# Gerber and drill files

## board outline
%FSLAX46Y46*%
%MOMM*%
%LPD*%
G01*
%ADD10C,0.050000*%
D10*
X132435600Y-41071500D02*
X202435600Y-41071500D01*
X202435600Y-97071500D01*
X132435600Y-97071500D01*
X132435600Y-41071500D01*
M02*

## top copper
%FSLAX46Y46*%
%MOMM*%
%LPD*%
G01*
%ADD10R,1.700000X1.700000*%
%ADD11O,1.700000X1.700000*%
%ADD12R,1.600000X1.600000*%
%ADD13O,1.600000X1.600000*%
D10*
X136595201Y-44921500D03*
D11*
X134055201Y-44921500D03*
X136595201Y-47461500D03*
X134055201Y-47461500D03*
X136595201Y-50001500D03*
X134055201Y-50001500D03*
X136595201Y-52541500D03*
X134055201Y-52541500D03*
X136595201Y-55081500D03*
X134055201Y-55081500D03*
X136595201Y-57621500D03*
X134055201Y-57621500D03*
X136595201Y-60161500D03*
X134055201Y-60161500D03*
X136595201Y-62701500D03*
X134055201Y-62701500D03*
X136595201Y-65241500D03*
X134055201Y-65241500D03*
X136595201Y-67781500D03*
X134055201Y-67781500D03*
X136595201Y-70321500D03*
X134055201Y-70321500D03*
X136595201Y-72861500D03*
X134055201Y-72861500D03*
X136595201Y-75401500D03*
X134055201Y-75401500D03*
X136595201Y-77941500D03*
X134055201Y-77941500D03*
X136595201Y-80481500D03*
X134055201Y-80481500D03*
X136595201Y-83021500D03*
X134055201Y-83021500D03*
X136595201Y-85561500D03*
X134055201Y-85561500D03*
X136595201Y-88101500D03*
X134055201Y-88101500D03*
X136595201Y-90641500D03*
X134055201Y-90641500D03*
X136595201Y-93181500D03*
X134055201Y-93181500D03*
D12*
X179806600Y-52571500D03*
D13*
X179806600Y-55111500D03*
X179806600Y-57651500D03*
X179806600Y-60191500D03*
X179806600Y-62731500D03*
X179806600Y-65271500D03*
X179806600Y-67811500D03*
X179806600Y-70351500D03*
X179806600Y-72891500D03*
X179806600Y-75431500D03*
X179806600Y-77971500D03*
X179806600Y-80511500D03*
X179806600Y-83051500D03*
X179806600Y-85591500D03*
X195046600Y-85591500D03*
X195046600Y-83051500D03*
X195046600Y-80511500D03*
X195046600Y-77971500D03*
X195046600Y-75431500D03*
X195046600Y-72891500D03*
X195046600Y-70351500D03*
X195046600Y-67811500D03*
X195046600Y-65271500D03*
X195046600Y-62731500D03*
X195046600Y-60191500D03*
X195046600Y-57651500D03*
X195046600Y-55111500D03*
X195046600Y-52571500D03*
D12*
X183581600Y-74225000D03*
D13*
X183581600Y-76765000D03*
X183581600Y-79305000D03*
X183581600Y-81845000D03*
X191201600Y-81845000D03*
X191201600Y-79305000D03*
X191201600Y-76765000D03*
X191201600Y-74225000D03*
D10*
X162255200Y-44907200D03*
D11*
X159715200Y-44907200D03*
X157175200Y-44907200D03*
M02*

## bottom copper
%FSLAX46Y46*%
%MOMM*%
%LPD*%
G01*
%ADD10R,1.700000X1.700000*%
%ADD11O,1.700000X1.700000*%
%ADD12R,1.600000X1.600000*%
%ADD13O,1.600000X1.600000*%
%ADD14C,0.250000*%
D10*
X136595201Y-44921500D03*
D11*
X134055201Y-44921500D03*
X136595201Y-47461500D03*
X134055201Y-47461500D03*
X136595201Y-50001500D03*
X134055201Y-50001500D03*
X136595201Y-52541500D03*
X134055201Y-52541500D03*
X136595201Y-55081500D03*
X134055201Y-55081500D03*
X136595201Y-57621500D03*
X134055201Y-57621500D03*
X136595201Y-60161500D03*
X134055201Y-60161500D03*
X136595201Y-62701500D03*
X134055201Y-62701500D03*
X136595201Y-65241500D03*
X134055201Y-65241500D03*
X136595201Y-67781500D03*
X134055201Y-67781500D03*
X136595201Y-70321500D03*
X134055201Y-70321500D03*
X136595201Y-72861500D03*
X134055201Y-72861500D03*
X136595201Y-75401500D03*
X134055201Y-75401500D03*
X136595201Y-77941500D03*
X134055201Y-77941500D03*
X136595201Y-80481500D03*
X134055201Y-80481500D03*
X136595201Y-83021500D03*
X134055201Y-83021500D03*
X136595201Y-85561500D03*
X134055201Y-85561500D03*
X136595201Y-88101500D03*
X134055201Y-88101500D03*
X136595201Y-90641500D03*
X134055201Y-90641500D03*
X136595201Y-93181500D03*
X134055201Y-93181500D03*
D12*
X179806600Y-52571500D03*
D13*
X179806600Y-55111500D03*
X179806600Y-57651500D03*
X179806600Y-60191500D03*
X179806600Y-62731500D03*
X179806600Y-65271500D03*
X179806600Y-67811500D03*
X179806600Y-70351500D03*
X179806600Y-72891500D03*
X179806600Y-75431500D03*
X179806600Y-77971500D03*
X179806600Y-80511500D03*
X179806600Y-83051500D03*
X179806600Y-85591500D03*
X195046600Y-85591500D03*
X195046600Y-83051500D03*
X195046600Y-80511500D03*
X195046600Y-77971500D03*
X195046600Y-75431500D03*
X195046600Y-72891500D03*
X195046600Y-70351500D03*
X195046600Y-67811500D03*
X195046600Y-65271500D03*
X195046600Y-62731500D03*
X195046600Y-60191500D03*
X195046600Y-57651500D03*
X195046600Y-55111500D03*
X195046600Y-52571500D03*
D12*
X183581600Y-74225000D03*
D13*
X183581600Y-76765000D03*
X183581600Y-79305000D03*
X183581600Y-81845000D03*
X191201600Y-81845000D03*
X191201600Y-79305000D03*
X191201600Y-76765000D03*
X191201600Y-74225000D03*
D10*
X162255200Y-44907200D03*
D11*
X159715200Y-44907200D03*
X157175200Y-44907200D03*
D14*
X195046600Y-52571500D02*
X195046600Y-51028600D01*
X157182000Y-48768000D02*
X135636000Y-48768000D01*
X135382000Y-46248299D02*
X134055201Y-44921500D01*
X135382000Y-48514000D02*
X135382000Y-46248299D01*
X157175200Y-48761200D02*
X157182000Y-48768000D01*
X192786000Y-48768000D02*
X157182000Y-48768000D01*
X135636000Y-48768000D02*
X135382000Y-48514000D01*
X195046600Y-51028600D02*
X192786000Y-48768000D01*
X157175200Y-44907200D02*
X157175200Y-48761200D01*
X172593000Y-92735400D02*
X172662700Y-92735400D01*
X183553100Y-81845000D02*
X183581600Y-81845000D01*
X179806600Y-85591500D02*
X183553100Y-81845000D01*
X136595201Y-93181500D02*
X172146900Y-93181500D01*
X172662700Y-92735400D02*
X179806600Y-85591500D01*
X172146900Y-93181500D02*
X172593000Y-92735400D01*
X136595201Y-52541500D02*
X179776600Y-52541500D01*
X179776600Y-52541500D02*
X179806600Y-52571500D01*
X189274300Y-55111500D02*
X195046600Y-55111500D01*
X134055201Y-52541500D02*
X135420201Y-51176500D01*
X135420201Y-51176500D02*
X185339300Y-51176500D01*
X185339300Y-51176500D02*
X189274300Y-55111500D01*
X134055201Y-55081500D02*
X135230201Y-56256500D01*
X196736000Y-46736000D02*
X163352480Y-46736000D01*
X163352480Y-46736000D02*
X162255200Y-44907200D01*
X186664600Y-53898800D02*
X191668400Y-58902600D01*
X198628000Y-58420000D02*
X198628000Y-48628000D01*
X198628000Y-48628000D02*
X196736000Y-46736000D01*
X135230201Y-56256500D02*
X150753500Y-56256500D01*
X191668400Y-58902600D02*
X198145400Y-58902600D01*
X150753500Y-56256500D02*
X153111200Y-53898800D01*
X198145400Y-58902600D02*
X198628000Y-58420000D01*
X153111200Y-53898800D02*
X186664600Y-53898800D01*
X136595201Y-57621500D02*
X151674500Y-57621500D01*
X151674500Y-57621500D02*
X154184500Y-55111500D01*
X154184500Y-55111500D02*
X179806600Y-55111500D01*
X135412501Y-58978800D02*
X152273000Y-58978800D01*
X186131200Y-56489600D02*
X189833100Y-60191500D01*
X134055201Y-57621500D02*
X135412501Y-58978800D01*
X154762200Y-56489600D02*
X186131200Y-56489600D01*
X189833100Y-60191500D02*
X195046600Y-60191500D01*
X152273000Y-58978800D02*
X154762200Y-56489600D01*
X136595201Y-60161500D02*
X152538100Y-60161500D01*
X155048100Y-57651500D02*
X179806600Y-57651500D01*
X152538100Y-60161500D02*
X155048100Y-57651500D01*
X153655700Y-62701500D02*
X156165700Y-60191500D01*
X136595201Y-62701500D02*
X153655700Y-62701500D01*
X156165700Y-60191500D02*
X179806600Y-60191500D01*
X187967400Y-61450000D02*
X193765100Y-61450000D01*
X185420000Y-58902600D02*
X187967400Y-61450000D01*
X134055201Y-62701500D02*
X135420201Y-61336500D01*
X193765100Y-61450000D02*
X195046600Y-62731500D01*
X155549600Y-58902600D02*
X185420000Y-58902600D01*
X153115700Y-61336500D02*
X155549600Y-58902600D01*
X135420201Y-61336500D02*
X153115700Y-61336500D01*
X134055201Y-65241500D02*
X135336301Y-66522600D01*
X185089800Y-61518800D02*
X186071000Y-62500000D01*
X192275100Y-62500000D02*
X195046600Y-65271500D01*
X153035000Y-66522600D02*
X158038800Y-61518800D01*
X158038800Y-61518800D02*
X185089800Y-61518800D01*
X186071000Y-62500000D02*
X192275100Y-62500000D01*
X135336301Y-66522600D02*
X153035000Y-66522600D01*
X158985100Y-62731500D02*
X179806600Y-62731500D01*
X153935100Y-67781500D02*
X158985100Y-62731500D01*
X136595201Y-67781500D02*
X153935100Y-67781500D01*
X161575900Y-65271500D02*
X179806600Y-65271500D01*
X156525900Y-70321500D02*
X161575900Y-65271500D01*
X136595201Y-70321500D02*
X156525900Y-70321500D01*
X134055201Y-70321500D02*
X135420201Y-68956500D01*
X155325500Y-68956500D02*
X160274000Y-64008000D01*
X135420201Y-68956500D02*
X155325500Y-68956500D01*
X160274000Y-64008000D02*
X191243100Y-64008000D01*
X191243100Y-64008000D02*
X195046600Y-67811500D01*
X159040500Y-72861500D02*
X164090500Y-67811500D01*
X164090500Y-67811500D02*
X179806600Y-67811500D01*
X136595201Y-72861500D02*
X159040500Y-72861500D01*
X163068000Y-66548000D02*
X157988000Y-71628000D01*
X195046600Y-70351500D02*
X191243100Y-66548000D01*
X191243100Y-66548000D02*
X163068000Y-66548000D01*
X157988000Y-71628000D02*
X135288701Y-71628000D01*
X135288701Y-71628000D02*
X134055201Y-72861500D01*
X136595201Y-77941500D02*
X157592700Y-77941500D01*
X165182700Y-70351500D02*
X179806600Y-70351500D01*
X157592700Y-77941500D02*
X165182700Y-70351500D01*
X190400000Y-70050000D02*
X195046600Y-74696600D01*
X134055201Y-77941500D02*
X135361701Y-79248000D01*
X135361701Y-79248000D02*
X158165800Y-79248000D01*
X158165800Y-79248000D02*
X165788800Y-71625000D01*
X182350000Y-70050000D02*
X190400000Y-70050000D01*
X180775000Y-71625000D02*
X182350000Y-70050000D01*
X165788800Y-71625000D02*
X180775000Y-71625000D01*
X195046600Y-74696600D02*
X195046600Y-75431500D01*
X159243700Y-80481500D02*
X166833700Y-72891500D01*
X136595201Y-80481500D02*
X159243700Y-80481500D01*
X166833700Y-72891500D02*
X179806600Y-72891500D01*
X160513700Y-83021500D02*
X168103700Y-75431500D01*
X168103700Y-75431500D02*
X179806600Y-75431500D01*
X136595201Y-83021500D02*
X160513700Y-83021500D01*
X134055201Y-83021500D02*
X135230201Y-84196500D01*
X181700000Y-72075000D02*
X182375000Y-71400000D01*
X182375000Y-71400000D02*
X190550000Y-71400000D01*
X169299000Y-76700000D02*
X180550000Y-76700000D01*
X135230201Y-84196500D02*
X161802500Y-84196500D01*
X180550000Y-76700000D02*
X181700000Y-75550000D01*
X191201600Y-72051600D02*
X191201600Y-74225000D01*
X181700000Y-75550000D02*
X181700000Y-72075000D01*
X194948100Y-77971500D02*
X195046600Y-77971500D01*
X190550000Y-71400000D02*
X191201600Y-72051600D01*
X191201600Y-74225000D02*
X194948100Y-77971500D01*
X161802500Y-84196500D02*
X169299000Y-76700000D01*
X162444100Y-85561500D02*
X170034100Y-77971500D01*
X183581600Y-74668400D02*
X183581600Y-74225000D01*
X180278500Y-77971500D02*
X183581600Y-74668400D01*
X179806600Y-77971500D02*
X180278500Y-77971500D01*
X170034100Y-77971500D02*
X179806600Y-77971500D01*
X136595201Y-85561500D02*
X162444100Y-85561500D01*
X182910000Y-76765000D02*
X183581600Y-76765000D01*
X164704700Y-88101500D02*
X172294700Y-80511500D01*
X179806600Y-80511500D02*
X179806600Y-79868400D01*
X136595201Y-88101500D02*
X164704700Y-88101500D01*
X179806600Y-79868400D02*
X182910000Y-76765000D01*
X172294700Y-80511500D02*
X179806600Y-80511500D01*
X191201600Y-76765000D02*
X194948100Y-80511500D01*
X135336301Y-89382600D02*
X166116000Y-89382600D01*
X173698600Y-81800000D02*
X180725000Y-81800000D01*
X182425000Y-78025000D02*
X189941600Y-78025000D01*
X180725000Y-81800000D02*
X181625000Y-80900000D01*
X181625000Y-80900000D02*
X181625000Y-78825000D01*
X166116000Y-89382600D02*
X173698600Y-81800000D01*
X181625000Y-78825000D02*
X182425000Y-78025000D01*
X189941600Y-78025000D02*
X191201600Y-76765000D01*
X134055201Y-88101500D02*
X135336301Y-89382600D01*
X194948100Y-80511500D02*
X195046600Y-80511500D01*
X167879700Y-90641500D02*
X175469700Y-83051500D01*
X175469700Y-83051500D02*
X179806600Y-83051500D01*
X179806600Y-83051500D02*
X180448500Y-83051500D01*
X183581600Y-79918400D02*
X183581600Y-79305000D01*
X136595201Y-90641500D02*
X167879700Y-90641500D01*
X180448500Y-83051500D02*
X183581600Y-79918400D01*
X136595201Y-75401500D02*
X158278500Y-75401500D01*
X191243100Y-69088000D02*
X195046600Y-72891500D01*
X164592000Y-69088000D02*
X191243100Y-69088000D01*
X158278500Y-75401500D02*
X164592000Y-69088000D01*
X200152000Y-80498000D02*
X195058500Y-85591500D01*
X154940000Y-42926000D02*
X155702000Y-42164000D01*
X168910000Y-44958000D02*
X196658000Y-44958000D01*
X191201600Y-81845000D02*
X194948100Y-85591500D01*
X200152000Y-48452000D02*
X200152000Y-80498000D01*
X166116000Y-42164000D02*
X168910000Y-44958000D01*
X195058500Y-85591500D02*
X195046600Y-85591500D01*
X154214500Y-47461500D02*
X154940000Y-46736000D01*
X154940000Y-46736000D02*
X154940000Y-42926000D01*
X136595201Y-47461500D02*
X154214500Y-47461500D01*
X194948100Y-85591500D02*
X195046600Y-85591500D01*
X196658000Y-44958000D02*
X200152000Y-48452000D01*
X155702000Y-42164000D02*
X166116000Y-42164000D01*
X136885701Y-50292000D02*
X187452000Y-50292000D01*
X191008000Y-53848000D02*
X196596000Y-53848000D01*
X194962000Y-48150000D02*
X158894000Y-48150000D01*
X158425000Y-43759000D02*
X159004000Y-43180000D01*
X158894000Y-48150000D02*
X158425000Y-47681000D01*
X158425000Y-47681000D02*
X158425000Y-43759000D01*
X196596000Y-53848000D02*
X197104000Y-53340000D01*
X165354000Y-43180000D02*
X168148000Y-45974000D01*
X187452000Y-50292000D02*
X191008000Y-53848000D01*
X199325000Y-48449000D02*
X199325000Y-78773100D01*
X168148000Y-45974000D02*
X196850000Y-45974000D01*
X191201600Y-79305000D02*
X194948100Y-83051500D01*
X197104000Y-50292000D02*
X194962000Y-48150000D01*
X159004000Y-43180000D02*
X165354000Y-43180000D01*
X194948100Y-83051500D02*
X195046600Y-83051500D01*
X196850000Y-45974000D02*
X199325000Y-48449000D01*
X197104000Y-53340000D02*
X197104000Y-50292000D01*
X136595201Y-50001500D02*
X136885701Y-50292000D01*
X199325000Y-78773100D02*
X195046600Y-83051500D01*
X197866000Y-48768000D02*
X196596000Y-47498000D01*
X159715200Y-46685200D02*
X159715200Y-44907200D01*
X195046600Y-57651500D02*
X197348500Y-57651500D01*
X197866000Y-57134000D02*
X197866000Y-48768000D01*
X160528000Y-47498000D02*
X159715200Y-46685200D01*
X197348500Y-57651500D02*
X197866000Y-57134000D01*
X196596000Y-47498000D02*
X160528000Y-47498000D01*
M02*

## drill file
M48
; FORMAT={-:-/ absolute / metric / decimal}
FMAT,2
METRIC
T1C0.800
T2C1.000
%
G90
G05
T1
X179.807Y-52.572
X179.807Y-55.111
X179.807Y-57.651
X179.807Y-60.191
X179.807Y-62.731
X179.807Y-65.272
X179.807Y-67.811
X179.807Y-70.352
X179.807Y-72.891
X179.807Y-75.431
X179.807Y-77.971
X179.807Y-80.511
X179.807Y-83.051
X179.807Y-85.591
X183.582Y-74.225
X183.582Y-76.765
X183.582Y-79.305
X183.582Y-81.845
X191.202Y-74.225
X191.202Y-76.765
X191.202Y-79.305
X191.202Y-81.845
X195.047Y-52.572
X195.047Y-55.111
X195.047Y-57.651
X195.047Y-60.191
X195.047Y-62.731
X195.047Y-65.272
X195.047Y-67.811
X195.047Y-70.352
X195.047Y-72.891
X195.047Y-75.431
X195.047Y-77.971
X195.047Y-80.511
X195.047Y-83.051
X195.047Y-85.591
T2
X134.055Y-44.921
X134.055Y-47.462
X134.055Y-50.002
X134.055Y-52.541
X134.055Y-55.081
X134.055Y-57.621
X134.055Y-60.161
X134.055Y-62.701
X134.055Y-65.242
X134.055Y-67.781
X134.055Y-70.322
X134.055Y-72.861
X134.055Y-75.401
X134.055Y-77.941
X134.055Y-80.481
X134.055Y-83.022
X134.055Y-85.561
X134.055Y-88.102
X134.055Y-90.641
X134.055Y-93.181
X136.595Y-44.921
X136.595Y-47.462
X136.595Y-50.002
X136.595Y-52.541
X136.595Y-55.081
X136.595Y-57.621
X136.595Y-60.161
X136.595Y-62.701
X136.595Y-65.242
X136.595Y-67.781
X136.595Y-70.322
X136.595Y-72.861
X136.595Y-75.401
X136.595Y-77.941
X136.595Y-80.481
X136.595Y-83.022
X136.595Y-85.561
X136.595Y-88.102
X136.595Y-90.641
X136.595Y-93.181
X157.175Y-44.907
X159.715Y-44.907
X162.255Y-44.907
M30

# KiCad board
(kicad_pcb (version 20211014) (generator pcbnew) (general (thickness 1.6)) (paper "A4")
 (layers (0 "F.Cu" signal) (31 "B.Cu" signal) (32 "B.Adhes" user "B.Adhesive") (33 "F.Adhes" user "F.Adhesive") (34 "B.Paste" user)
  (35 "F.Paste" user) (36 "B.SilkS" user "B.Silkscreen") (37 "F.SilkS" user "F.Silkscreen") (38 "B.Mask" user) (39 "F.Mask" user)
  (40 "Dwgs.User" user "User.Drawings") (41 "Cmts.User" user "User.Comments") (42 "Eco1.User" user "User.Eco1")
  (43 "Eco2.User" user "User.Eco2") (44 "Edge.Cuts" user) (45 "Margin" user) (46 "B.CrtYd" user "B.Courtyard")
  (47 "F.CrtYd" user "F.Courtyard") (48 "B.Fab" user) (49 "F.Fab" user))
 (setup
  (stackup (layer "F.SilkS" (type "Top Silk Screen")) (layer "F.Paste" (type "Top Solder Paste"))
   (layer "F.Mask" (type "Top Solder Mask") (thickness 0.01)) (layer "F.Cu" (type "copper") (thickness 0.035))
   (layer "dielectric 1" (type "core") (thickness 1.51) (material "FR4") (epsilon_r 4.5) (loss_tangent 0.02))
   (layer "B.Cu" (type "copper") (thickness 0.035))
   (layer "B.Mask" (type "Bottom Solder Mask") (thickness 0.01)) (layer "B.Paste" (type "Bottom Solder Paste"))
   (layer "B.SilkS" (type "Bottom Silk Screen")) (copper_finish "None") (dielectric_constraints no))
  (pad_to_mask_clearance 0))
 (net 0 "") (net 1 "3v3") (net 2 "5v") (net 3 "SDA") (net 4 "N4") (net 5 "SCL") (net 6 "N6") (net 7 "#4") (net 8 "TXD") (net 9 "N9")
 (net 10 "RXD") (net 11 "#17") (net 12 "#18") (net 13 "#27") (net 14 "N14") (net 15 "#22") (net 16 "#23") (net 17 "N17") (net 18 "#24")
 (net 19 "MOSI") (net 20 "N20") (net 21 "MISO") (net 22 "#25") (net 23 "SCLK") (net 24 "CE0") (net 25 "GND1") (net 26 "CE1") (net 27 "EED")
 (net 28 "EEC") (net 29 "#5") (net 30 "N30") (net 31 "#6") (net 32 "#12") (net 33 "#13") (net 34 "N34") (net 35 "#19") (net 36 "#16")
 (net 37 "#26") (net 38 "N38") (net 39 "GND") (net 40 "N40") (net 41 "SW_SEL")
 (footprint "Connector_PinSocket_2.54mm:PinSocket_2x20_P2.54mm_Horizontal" (layer "F.Cu") (at 136.595201 44.9215)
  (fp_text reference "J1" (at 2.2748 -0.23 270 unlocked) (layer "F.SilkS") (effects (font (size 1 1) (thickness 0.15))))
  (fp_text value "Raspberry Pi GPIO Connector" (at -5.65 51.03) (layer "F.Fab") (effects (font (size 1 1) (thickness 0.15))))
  (pad "1" thru_hole rect (at 0 0) (size 1.7 1.7) (drill 1) (layers *.Cu *.Mask) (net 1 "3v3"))
  (pad "2" thru_hole oval (at -2.54 0) (size 1.7 1.7) (drill 1) (layers *.Cu *.Mask) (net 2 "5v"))
  (pad "3" thru_hole oval (at 0 2.54) (size 1.7 1.7) (drill 1) (layers *.Cu *.Mask) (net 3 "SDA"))
  (pad "4" thru_hole oval (at -2.54 2.54) (size 1.7 1.7) (drill 1) (layers *.Cu *.Mask) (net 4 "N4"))
  (pad "5" thru_hole oval (at 0 5.08) (size 1.7 1.7) (drill 1) (layers *.Cu *.Mask) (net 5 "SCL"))
  (pad "6" thru_hole oval (at -2.54 5.08) (size 1.7 1.7) (drill 1) (layers *.Cu *.Mask) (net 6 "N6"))
  (pad "7" thru_hole oval (at 0 7.62) (size 1.7 1.7) (drill 1) (layers *.Cu *.Mask) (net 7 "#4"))
  (pad "8" thru_hole oval (at -2.54 7.62) (size 1.7 1.7) (drill 1) (layers *.Cu *.Mask) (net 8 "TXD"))
  (pad "9" thru_hole oval (at 0 10.16) (size 1.7 1.7) (drill 1) (layers *.Cu *.Mask) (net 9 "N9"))
  (pad "10" thru_hole oval (at -2.54 10.16) (size 1.7 1.7) (drill 1) (layers *.Cu *.Mask) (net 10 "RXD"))
  (pad "11" thru_hole oval (at 0 12.7) (size 1.7 1.7) (drill 1) (layers *.Cu *.Mask) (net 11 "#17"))
  (pad "12" thru_hole oval (at -2.54 12.7) (size 1.7 1.7) (drill 1) (layers *.Cu *.Mask) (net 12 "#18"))
  (pad "13" thru_hole oval (at 0 15.24) (size 1.7 1.7) (drill 1) (layers *.Cu *.Mask) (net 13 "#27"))
  (pad "14" thru_hole oval (at -2.54 15.24) (size 1.7 1.7) (drill 1) (layers *.Cu *.Mask) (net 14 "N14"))
  (pad "15" thru_hole oval (at 0 17.78) (size 1.7 1.7) (drill 1) (layers *.Cu *.Mask) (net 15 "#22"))
  (pad "16" thru_hole oval (at -2.54 17.78) (size 1.7 1.7) (drill 1) (layers *.Cu *.Mask) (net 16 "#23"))
  (pad "17" thru_hole oval (at 0 20.32) (size 1.7 1.7) (drill 1) (layers *.Cu *.Mask) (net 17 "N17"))
  (pad "18" thru_hole oval (at -2.54 20.32) (size 1.7 1.7) (drill 1) (layers *.Cu *.Mask) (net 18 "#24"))
  (pad "19" thru_hole oval (at 0 22.86) (size 1.7 1.7) (drill 1) (layers *.Cu *.Mask) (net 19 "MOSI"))
  (pad "20" thru_hole oval (at -2.54 22.86) (size 1.7 1.7) (drill 1) (layers *.Cu *.Mask) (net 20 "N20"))
  (pad "21" thru_hole oval (at 0 25.4) (size 1.7 1.7) (drill 1) (layers *.Cu *.Mask) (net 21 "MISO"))
  (pad "22" thru_hole oval (at -2.54 25.4) (size 1.7 1.7) (drill 1) (layers *.Cu *.Mask) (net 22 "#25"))
  (pad "23" thru_hole oval (at 0 27.94) (size 1.7 1.7) (drill 1) (layers *.Cu *.Mask) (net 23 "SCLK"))
  (pad "24" thru_hole oval (at -2.54 27.94) (size 1.7 1.7) (drill 1) (layers *.Cu *.Mask) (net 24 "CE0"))
  (pad "25" thru_hole oval (at 0 30.48) (size 1.7 1.7) (drill 1) (layers *.Cu *.Mask) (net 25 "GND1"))
  (pad "26" thru_hole oval (at -2.54 30.48) (size 1.7 1.7) (drill 1) (layers *.Cu *.Mask) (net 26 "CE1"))
  (pad "27" thru_hole oval (at 0 33.02) (size 1.7 1.7) (drill 1) (layers *.Cu *.Mask) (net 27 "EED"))
  (pad "28" thru_hole oval (at -2.54 33.02) (size 1.7 1.7) (drill 1) (layers *.Cu *.Mask) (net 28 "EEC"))
  (pad "29" thru_hole oval (at 0 35.56) (size 1.7 1.7) (drill 1) (layers *.Cu *.Mask) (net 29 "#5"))
  (pad "30" thru_hole oval (at -2.54 35.56) (size 1.7 1.7) (drill 1) (layers *.Cu *.Mask) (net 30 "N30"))
  (pad "31" thru_hole oval (at 0 38.1) (size 1.7 1.7) (drill 1) (layers *.Cu *.Mask) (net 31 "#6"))
  (pad "32" thru_hole oval (at -2.54 38.1) (size 1.7 1.7) (drill 1) (layers *.Cu *.Mask) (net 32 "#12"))
  (pad "33" thru_hole oval (at 0 40.64) (size 1.7 1.7) (drill 1) (layers *.Cu *.Mask) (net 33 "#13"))
  (pad "34" thru_hole oval (at -2.54 40.64) (size 1.7 1.7) (drill 1) (layers *.Cu *.Mask) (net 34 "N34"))
  (pad "35" thru_hole oval (at 0 43.18) (size 1.7 1.7) (drill 1) (layers *.Cu *.Mask) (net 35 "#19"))
  (pad "36" thru_hole oval (at -2.54 43.18) (size 1.7 1.7) (drill 1) (layers *.Cu *.Mask) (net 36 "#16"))
  (pad "37" thru_hole oval (at 0 45.72) (size 1.7 1.7) (drill 1) (layers *.Cu *.Mask) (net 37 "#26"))
  (pad "38" thru_hole oval (at -2.54 45.72) (size 1.7 1.7) (drill 1) (layers *.Cu *.Mask) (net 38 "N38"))
  (pad "39" thru_hole oval (at 0 48.26) (size 1.7 1.7) (drill 1) (layers *.Cu *.Mask) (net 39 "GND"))
  (pad "40" thru_hole oval (at -2.54 48.26) (size 1.7 1.7) (drill 1) (layers *.Cu *.Mask) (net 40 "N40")))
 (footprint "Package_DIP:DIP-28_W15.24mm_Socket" (layer "F.Cu") (at 179.8066 52.5715)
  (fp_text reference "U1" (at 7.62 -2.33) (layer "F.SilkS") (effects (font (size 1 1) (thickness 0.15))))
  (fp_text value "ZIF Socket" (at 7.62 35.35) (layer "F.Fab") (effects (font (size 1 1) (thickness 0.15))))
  (pad "1" thru_hole rect (at 0 0) (size 1.6 1.6) (drill 0.8) (layers *.Cu *.Mask) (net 7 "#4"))
  (pad "2" thru_hole oval (at 0 2.54) (size 1.6 1.6) (drill 0.8) (layers *.Cu *.Mask) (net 11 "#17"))
  (pad "3" thru_hole oval (at 0 5.08) (size 1.6 1.6) (drill 0.8) (layers *.Cu *.Mask) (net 13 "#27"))
  (pad "4" thru_hole oval (at 0 7.62) (size 1.6 1.6) (drill 0.8) (layers *.Cu *.Mask) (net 15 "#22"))
  (pad "5" thru_hole oval (at 0 10.16) (size 1.6 1.6) (drill 0.8) (layers *.Cu *.Mask) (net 19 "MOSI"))
  (pad "6" thru_hole oval (at 0 12.7) (size 1.6 1.6) (drill 0.8) (layers *.Cu *.Mask) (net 21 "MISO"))
  (pad "7" thru_hole oval (at 0 15.24) (size 1.6 1.6) (drill 0.8) (layers *.Cu *.Mask) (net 23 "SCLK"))
  (pad "8" thru_hole oval (at 0 17.78) (size 1.6 1.6) (drill 0.8) (layers *.Cu *.Mask) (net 27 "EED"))
  (pad "9" thru_hole oval (at 0 20.32) (size 1.6 1.6) (drill 0.8) (layers *.Cu *.Mask) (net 29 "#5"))
  (pad "10" thru_hole oval (at 0 22.86) (size 1.6 1.6) (drill 0.8) (layers *.Cu *.Mask) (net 31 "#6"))
  (pad "11" thru_hole oval (at 0 25.4) (size 1.6 1.6) (drill 0.8) (layers *.Cu *.Mask) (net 33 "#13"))
  (pad "12" thru_hole oval (at 0 27.94) (size 1.6 1.6) (drill 0.8) (layers *.Cu *.Mask) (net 35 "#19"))
  (pad "13" thru_hole oval (at 0 30.48) (size 1.6 1.6) (drill 0.8) (layers *.Cu *.Mask) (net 37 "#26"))
  (pad "14" thru_hole oval (at 0 33.02) (size 1.6 1.6) (drill 0.8) (layers *.Cu *.Mask) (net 39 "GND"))
  (pad "15" thru_hole oval (at 15.24 33.02) (size 1.6 1.6) (drill 0.8) (layers *.Cu *.Mask) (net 3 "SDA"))
  (pad "16" thru_hole oval (at 15.24 30.48) (size 1.6 1.6) (drill 0.8) (layers *.Cu *.Mask) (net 5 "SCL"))
  (pad "17" thru_hole oval (at 15.24 27.94) (size 1.6 1.6) (drill 0.8) (layers *.Cu *.Mask) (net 36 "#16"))
  (pad "18" thru_hole oval (at 15.24 25.4) (size 1.6 1.6) (drill 0.8) (layers *.Cu *.Mask) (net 32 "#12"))
  (pad "19" thru_hole oval (at 15.24 22.86) (size 1.6 1.6) (drill 0.8) (layers *.Cu *.Mask) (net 28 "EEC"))
  (pad "20" thru_hole oval (at 15.24 20.32) (size 1.6 1.6) (drill 0.8) (layers *.Cu *.Mask) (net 25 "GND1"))
  (pad "21" thru_hole oval (at 15.24 17.78) (size 1.6 1.6) (drill 0.8) (layers *.Cu *.Mask) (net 24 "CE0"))
  (pad "22" thru_hole oval (at 15.24 15.24) (size 1.6 1.6) (drill 0.8) (layers *.Cu *.Mask) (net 22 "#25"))
  (pad "23" thru_hole oval (at 15.24 12.7) (size 1.6 1.6) (drill 0.8) (layers *.Cu *.Mask) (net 18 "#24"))
  (pad "24" thru_hole oval (at 15.24 10.16) (size 1.6 1.6) (drill 0.8) (layers *.Cu *.Mask) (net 16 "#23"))
  (pad "25" thru_hole oval (at 15.24 7.62) (size 1.6 1.6) (drill 0.8) (layers *.Cu *.Mask) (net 12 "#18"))
  (pad "26" thru_hole oval (at 15.24 5.08) (size 1.6 1.6) (drill 0.8) (layers *.Cu *.Mask) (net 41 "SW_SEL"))
  (pad "27" thru_hole oval (at 15.24 2.54) (size 1.6 1.6) (drill 0.8) (layers *.Cu *.Mask) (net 8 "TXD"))
  (pad "28" thru_hole oval (at 15.24 0) (size 1.6 1.6) (drill 0.8) (layers *.Cu *.Mask) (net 2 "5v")))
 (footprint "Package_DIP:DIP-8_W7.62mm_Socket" (layer "F.Cu") (at 183.5816 74.225)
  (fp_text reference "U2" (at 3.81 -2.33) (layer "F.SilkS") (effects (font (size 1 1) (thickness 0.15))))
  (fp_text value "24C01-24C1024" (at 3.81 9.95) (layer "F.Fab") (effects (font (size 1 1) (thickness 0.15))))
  (pad "1" thru_hole rect (at 0 0) (size 1.6 1.6) (drill 0.8) (layers *.Cu *.Mask) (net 33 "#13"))
  (pad "2" thru_hole oval (at 0 2.54) (size 1.6 1.6) (drill 0.8) (layers *.Cu *.Mask) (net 35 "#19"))
  (pad "3" thru_hole oval (at 0 5.08) (size 1.6 1.6) (drill 0.8) (layers *.Cu *.Mask) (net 37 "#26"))
  (pad "4" thru_hole oval (at 0 7.62) (size 1.6 1.6) (drill 0.8) (layers *.Cu *.Mask) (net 39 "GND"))
  (pad "5" thru_hole oval (at 7.62 7.62) (size 1.6 1.6) (drill 0.8) (layers *.Cu *.Mask) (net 3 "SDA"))
  (pad "6" thru_hole oval (at 7.62 5.08) (size 1.6 1.6) (drill 0.8) (layers *.Cu *.Mask) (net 5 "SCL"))
  (pad "7" thru_hole oval (at 7.62 2.54) (size 1.6 1.6) (drill 0.8) (layers *.Cu *.Mask) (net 36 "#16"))
  (pad "8" thru_hole oval (at 7.62 0) (size 1.6 1.6) (drill 0.8) (layers *.Cu *.Mask) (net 32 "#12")))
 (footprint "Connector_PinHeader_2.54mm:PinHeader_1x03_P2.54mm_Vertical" (layer "F.Cu") (at 162.2552 44.9072 -90)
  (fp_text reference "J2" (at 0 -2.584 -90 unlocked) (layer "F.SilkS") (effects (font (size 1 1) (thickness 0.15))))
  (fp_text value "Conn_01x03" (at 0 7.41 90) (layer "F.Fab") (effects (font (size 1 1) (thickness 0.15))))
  (pad "1" thru_hole rect (at 0 0 270) (size 1.7 1.7) (drill 1) (layers *.Cu *.Mask) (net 10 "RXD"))
  (pad "2" thru_hole oval (at 0 2.54 270) (size 1.7 1.7) (drill 1) (layers *.Cu *.Mask) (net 41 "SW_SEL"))
  (pad "3" thru_hole oval (at 0 5.08 270) (size 1.7 1.7) (drill 1) (layers *.Cu *.Mask) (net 2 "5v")))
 (gr_rect (start 132.4356 41.0715) (end 202.4356 97.0715) (layer "Edge.Cuts") (width 0.05) (fill none))
 (segment (start 195.0466 52.5715) (end 195.0466 51.0286) (width 0.25) (layer "B.Cu") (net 2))
 (segment (start 157.182 48.768) (end 135.636 48.768) (width 0.25) (layer "B.Cu") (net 2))
 (segment (start 135.382 46.248299) (end 134.055201 44.9215) (width 0.25) (layer "B.Cu") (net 2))
 (segment (start 135.382 48.514) (end 135.382 46.248299) (width 0.25) (layer "B.Cu") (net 2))
 (segment (start 157.1752 48.7612) (end 157.182 48.768) (width 0.25) (layer "B.Cu") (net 2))
 (segment (start 192.786 48.768) (end 157.182 48.768) (width 0.25) (layer "B.Cu") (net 2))
 (segment (start 135.636 48.768) (end 135.382 48.514) (width 0.25) (layer "B.Cu") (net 2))
 (segment (start 195.0466 51.0286) (end 192.786 48.768) (width 0.25) (layer "B.Cu") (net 2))
 (segment (start 157.1752 44.9072) (end 157.1752 48.7612) (width 0.25) (layer "B.Cu") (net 2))
 (segment (start 172.593 92.7354) (end 172.6627 92.7354) (width 0.25) (layer "B.Cu") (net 39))
 (segment (start 183.5531 81.845) (end 183.5816 81.845) (width 0.25) (layer "B.Cu") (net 39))
 (segment (start 179.8066 85.5915) (end 183.5531 81.845) (width 0.25) (layer "B.Cu") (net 39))
 (segment (start 136.595201 93.1815) (end 172.1469 93.1815) (width 0.25) (layer "B.Cu") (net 39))
 (segment (start 172.6627 92.7354) (end 179.8066 85.5915) (width 0.25) (layer "B.Cu") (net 39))
 (segment (start 172.1469 93.1815) (end 172.593 92.7354) (width 0.25) (layer "B.Cu") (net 39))
 (segment (start 136.595201 52.5415) (end 179.7766 52.5415) (width 0.25) (layer "B.Cu") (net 7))
 (segment (start 179.7766 52.5415) (end 179.8066 52.5715) (width 0.25) (layer "B.Cu") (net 7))
 (segment (start 189.2743 55.1115) (end 195.0466 55.1115) (width 0.25) (layer "B.Cu") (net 8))
 (segment (start 134.055201 52.5415) (end 135.420201 51.1765) (width 0.25) (layer "B.Cu") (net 8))
 (segment (start 135.420201 51.1765) (end 185.3393 51.1765) (width 0.25) (layer "B.Cu") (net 8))
 (segment (start 185.3393 51.1765) (end 189.2743 55.1115) (width 0.25) (layer "B.Cu") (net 8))
 (segment (start 134.055201 55.0815) (end 135.230201 56.2565) (width 0.25) (layer "B.Cu") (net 10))
 (segment (start 196.736 46.736) (end 163.35248 46.736) (width 0.25) (layer "B.Cu") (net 10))
 (segment (start 163.35248 46.736) (end 162.2552 44.9072) (width 0.25) (layer "B.Cu") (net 10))
 (segment (start 186.6646 53.8988) (end 191.6684 58.9026) (width 0.25) (layer "B.Cu") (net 10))
 (segment (start 198.628 58.42) (end 198.628 48.628) (width 0.25) (layer "B.Cu") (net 10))
 (segment (start 198.628 48.628) (end 196.736 46.736) (width 0.25) (layer "B.Cu") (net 10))
 (segment (start 135.230201 56.2565) (end 150.7535 56.2565) (width 0.25) (layer "B.Cu") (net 10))
 (segment (start 191.6684 58.9026) (end 198.1454 58.9026) (width 0.25) (layer "B.Cu") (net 10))
 (segment (start 150.7535 56.2565) (end 153.1112 53.8988) (width 0.25) (layer "B.Cu") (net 10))
 (segment (start 198.1454 58.9026) (end 198.628 58.42) (width 0.25) (layer "B.Cu") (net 10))
 (segment (start 153.1112 53.8988) (end 186.6646 53.8988) (width 0.25) (layer "B.Cu") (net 10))
 (segment (start 136.595201 57.6215) (end 151.6745 57.6215) (width 0.25) (layer "B.Cu") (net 11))
 (segment (start 151.6745 57.6215) (end 154.1845 55.1115) (width 0.25) (layer "B.Cu") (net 11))
 (segment (start 154.1845 55.1115) (end 179.8066 55.1115) (width 0.25) (layer "B.Cu") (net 11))
 (segment (start 135.412501 58.9788) (end 152.273 58.9788) (width 0.25) (layer "B.Cu") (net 12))
 (segment (start 186.1312 56.4896) (end 189.8331 60.1915) (width 0.25) (layer "B.Cu") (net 12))
 (segment (start 134.055201 57.6215) (end 135.412501 58.9788) (width 0.25) (layer "B.Cu") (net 12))
 (segment (start 154.7622 56.4896) (end 186.1312 56.4896) (width 0.25) (layer "B.Cu") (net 12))
 (segment (start 189.8331 60.1915) (end 195.0466 60.1915) (width 0.25) (layer "B.Cu") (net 12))
 (segment (start 152.273 58.9788) (end 154.7622 56.4896) (width 0.25) (layer "B.Cu") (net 12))
 (segment (start 136.595201 60.1615) (end 152.5381 60.1615) (width 0.25) (layer "B.Cu") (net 13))
 (segment (start 155.0481 57.6515) (end 179.8066 57.6515) (width 0.25) (layer "B.Cu") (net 13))
 (segment (start 152.5381 60.1615) (end 155.0481 57.6515) (width 0.25) (layer "B.Cu") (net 13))
 (segment (start 153.6557 62.7015) (end 156.1657 60.1915) (width 0.25) (layer "B.Cu") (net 15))
 (segment (start 136.595201 62.7015) (end 153.6557 62.7015) (width 0.25) (layer "B.Cu") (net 15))
 (segment (start 156.1657 60.1915) (end 179.8066 60.1915) (width 0.25) (layer "B.Cu") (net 15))
 (segment (start 187.9674 61.45) (end 193.7651 61.45) (width 0.25) (layer "B.Cu") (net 16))
 (segment (start 185.42 58.9026) (end 187.9674 61.45) (width 0.25) (layer "B.Cu") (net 16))
 (segment (start 134.055201 62.7015) (end 135.420201 61.3365) (width 0.25) (layer "B.Cu") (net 16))
 (segment (start 193.7651 61.45) (end 195.0466 62.7315) (width 0.25) (layer "B.Cu") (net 16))
 (segment (start 155.5496 58.9026) (end 185.42 58.9026) (width 0.25) (layer "B.Cu") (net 16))
 (segment (start 153.1157 61.3365) (end 155.5496 58.9026) (width 0.25) (layer "B.Cu") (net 16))
 (segment (start 135.420201 61.3365) (end 153.1157 61.3365) (width 0.25) (layer "B.Cu") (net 16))
 (segment (start 134.055201 65.2415) (end 135.336301 66.5226) (width 0.25) (layer "B.Cu") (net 18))
 (segment (start 185.0898 61.5188) (end 186.071 62.5) (width 0.25) (layer "B.Cu") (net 18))
 (segment (start 192.2751 62.5) (end 195.0466 65.2715) (width 0.25) (layer "B.Cu") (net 18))
 (segment (start 153.035 66.5226) (end 158.0388 61.5188) (width 0.25) (layer "B.Cu") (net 18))
 (segment (start 158.0388 61.5188) (end 185.0898 61.5188) (width 0.25) (layer "B.Cu") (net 18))
 (segment (start 186.071 62.5) (end 192.2751 62.5) (width 0.25) (layer "B.Cu") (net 18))
 (segment (start 135.336301 66.5226) (end 153.035 66.5226) (width 0.25) (layer "B.Cu") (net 18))
 (segment (start 158.9851 62.7315) (end 179.8066 62.7315) (width 0.25) (layer "B.Cu") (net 19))
 (segment (start 153.9351 67.7815) (end 158.9851 62.7315) (width 0.25) (layer "B.Cu") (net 19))
 (segment (start 136.595201 67.7815) (end 153.9351 67.7815) (width 0.25) (layer "B.Cu") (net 19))
 (segment (start 161.5759 65.2715) (end 179.8066 65.2715) (width 0.25) (layer "B.Cu") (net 21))
 (segment (start 156.5259 70.3215) (end 161.5759 65.2715) (width 0.25) (layer "B.Cu") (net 21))
 (segment (start 136.595201 70.3215) (end 156.5259 70.3215) (width 0.25) (layer "B.Cu") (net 21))
 (segment (start 134.055201 70.3215) (end 135.420201 68.9565) (width 0.25) (layer "B.Cu") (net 22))
 (segment (start 155.3255 68.9565) (end 160.274 64.008) (width 0.25) (layer "B.Cu") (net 22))
 (segment (start 135.420201 68.9565) (end 155.3255 68.9565) (width 0.25) (layer "B.Cu") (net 22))
 (segment (start 160.274 64.008) (end 191.2431 64.008) (width 0.25) (layer "B.Cu") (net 22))
 (segment (start 191.2431 64.008) (end 195.0466 67.8115) (width 0.25) (layer "B.Cu") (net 22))
 (segment (start 159.0405 72.8615) (end 164.0905 67.8115) (width 0.25) (layer "B.Cu") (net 23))
 (segment (start 164.0905 67.8115) (end 179.8066 67.8115) (width 0.25) (layer "B.Cu") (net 23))
 (segment (start 136.595201 72.8615) (end 159.0405 72.8615) (width 0.25) (layer "B.Cu") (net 23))
 (segment (start 163.068 66.548) (end 157.988 71.628) (width 0.25) (layer "B.Cu") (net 24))
 (segment (start 195.0466 70.3515) (end 191.2431 66.548) (width 0.25) (layer "B.Cu") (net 24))
 (segment (start 191.2431 66.548) (end 163.068 66.548) (width 0.25) (layer "B.Cu") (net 24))
 (segment (start 157.988 71.628) (end 135.288701 71.628) (width 0.25) (layer "B.Cu") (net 24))
 (segment (start 135.288701 71.628) (end 134.055201 72.8615) (width 0.25) (layer "B.Cu") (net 24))
 (segment (start 136.595201 77.9415) (end 157.5927 77.9415) (width 0.25) (layer "B.Cu") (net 27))
 (segment (start 165.1827 70.3515) (end 179.8066 70.3515) (width 0.25) (layer "B.Cu") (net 27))
 (segment (start 157.5927 77.9415) (end 165.1827 70.3515) (width 0.25) (layer "B.Cu") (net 27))
 (segment (start 190.4 70.05) (end 195.0466 74.6966) (width 0.25) (layer "B.Cu") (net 28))
 (segment (start 134.055201 77.9415) (end 135.361701 79.248) (width 0.25) (layer "B.Cu") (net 28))
 (segment (start 135.361701 79.248) (end 158.1658 79.248) (width 0.25) (layer "B.Cu") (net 28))
 (segment (start 158.1658 79.248) (end 165.7888 71.625) (width 0.25) (layer "B.Cu") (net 28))
 (segment (start 182.35 70.05) (end 190.4 70.05) (width 0.25) (layer "B.Cu") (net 28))
 (segment (start 180.775 71.625) (end 182.35 70.05) (width 0.25) (layer "B.Cu") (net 28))
 (segment (start 165.7888 71.625) (end 180.775 71.625) (width 0.25) (layer "B.Cu") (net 28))
 (segment (start 195.0466 74.6966) (end 195.0466 75.4315) (width 0.25) (layer "B.Cu") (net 28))
 (segment (start 159.2437 80.4815) (end 166.8337 72.8915) (width 0.25) (layer "B.Cu") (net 29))
 (segment (start 136.595201 80.4815) (end 159.2437 80.4815) (width 0.25) (layer "B.Cu") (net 29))
 (segment (start 166.8337 72.8915) (end 179.8066 72.8915) (width 0.25) (layer "B.Cu") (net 29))
 (segment (start 160.5137 83.0215) (end 168.1037 75.4315) (width 0.25) (layer "B.Cu") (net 31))
 (segment (start 168.1037 75.4315) (end 179.8066 75.4315) (width 0.25) (layer "B.Cu") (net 31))
 (segment (start 136.595201 83.0215) (end 160.5137 83.0215) (width 0.25) (layer "B.Cu") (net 31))
 (segment (start 134.055201 83.0215) (end 135.230201 84.1965) (width 0.25) (layer "B.Cu") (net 32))
 (segment (start 181.7 72.075) (end 182.375 71.4) (width 0.25) (layer "B.Cu") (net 32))
 (segment (start 182.375 71.4) (end 190.55 71.4) (width 0.25) (layer "B.Cu") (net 32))
 (segment (start 169.299 76.7) (end 180.55 76.7) (width 0.25) (layer "B.Cu") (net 32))
 (segment (start 135.230201 84.1965) (end 161.8025 84.1965) (width 0.25) (layer "B.Cu") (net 32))
 (segment (start 180.55 76.7) (end 181.7 75.55) (width 0.25) (layer "B.Cu") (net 32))
 (segment (start 191.2016 72.0516) (end 191.2016 74.225) (width 0.25) (layer "B.Cu") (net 32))
 (segment (start 181.7 75.55) (end 181.7 72.075) (width 0.25) (layer "B.Cu") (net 32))
 (segment (start 194.9481 77.9715) (end 195.0466 77.9715) (width 0.25) (layer "B.Cu") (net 32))
 (segment (start 190.55 71.4) (end 191.2016 72.0516) (width 0.25) (layer "B.Cu") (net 32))
 (segment (start 191.2016 74.225) (end 194.9481 77.9715) (width 0.25) (layer "B.Cu") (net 32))
 (segment (start 161.8025 84.1965) (end 169.299 76.7) (width 0.25) (layer "B.Cu") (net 32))
 (segment (start 162.4441 85.5615) (end 170.0341 77.9715) (width 0.25) (layer "B.Cu") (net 33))
 (segment (start 183.5816 74.6684) (end 183.5816 74.225) (width 0.25) (layer "B.Cu") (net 33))
 (segment (start 180.2785 77.9715) (end 183.5816 74.6684) (width 0.25) (layer "B.Cu") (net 33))
 (segment (start 179.8066 77.9715) (end 180.2785 77.9715) (width 0.25) (layer "B.Cu") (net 33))
 (segment (start 170.0341 77.9715) (end 179.8066 77.9715) (width 0.25) (layer "B.Cu") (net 33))
 (segment (start 136.595201 85.5615) (end 162.4441 85.5615) (width 0.25) (layer "B.Cu") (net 33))
 (segment (start 182.91 76.765) (end 183.5816 76.765) (width 0.25) (layer "B.Cu") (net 35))
 (segment (start 164.7047 88.1015) (end 172.2947 80.5115) (width 0.25) (layer "B.Cu") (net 35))
 (segment (start 179.8066 80.5115) (end 179.8066 79.8684) (width 0.25) (layer "B.Cu") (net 35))
 (segment (start 136.595201 88.1015) (end 164.7047 88.1015) (width 0.25) (layer "B.Cu") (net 35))
 (segment (start 179.8066 79.8684) (end 182.91 76.765) (width 0.25) (layer "B.Cu") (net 35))
 (segment (start 172.2947 80.5115) (end 179.8066 80.5115) (width 0.25) (layer "B.Cu") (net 35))
 (segment (start 191.2016 76.765) (end 194.9481 80.5115) (width 0.25) (layer "B.Cu") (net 36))
 (segment (start 135.336301 89.3826) (end 166.116 89.3826) (width 0.25) (layer "B.Cu") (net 36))
 (segment (start 173.6986 81.8) (end 180.725 81.8) (width 0.25) (layer "B.Cu") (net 36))
 (segment (start 182.425 78.025) (end 189.9416 78.025) (width 0.25) (layer "B.Cu") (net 36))
 (segment (start 180.725 81.8) (end 181.625 80.9) (width 0.25) (layer "B.Cu") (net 36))
 (segment (start 181.625 80.9) (end 181.625 78.825) (width 0.25) (layer "B.Cu") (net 36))
 (segment (start 166.116 89.3826) (end 173.6986 81.8) (width 0.25) (layer "B.Cu") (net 36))
 (segment (start 181.625 78.825) (end 182.425 78.025) (width 0.25) (layer "B.Cu") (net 36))
 (segment (start 189.9416 78.025) (end 191.2016 76.765) (width 0.25) (layer "B.Cu") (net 36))
 (segment (start 134.055201 88.1015) (end 135.336301 89.3826) (width 0.25) (layer "B.Cu") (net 36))
 (segment (start 194.9481 80.5115) (end 195.0466 80.5115) (width 0.25) (layer "B.Cu") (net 36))
 (segment (start 167.8797 90.6415) (end 175.4697 83.0515) (width 0.25) (layer "B.Cu") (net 37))
 (segment (start 175.4697 83.0515) (end 179.8066 83.0515) (width 0.25) (layer "B.Cu") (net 37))
 (segment (start 179.8066 83.0515) (end 180.4485 83.0515) (width 0.25) (layer "B.Cu") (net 37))
 (segment (start 183.5816 79.9184) (end 183.5816 79.305) (width 0.25) (layer "B.Cu") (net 37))
 (segment (start 136.595201 90.6415) (end 167.8797 90.6415) (width 0.25) (layer "B.Cu") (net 37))
 (segment (start 180.4485 83.0515) (end 183.5816 79.9184) (width 0.25) (layer "B.Cu") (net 37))
 (segment (start 136.595201 75.4015) (end 158.2785 75.4015) (width 0.25) (layer "B.Cu") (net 25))
 (segment (start 191.2431 69.088) (end 195.0466 72.8915) (width 0.25) (layer "B.Cu") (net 25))
 (segment (start 164.592 69.088) (end 191.2431 69.088) (width 0.25) (layer "B.Cu") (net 25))
 (segment (start 158.2785 75.4015) (end 164.592 69.088) (width 0.25) (layer "B.Cu") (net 25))
 (segment (start 200.152 80.498) (end 195.0585 85.5915) (width 0.25) (layer "B.Cu") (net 3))
 (segment (start 154.94 42.926) (end 155.702 42.164) (width 0.25) (layer "B.Cu") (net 3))
 (segment (start 168.91 44.958) (end 196.658 44.958) (width 0.25) (layer "B.Cu") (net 3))
 (segment (start 191.2016 81.845) (end 194.9481 85.5915) (width 0.25) (layer "B.Cu") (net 3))
 (segment (start 200.152 48.452) (end 200.152 80.498) (width 0.25) (layer "B.Cu") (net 3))
 (segment (start 166.116 42.164) (end 168.91 44.958) (width 0.25) (layer "B.Cu") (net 3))
 (segment (start 195.0585 85.5915) (end 195.0466 85.5915) (width 0.25) (layer "B.Cu") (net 3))
 (segment (start 154.2145 47.4615) (end 154.94 46.736) (width 0.25) (layer "B.Cu") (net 3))
 (segment (start 154.94 46.736) (end 154.94 42.926) (width 0.25) (layer "B.Cu") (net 3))
 (segment (start 136.595201 47.4615) (end 154.2145 47.4615) (width 0.25) (layer "B.Cu") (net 3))
 (segment (start 194.9481 85.5915) (end 195.0466 85.5915) (width 0.25) (layer "B.Cu") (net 3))
 (segment (start 196.658 44.958) (end 200.152 48.452) (width 0.25) (layer "B.Cu") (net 3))
 (segment (start 155.702 42.164) (end 166.116 42.164) (width 0.25) (layer "B.Cu") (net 3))
 (segment (start 136.885701 50.292) (end 187.452 50.292) (width 0.25) (layer "B.Cu") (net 5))
 (segment (start 191.008 53.848) (end 196.596 53.848) (width 0.25) (layer "B.Cu") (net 5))
 (segment (start 194.962 48.15) (end 158.894 48.15) (width 0.25) (layer "B.Cu") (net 5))
 (segment (start 158.425 43.759) (end 159.004 43.18) (width 0.25) (layer "B.Cu") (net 5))
 (segment (start 158.894 48.15) (end 158.425 47.681) (width 0.25) (layer "B.Cu") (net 5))
 (segment (start 158.425 47.681) (end 158.425 43.759) (width 0.25) (layer "B.Cu") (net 5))
 (segment (start 196.596 53.848) (end 197.104 53.34) (width 0.25) (layer "B.Cu") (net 5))
 (segment (start 165.354 43.18) (end 168.148 45.974) (width 0.25) (layer "B.Cu") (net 5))
 (segment (start 187.452 50.292) (end 191.008 53.848) (width 0.25) (layer "B.Cu") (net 5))
 (segment (start 199.325 48.449) (end 199.325 78.7731) (width 0.25) (layer "B.Cu") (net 5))
 (segment (start 168.148 45.974) (end 196.85 45.974) (width 0.25) (layer "B.Cu") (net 5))
 (segment (start 191.2016 79.305) (end 194.9481 83.0515) (width 0.25) (layer "B.Cu") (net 5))
 (segment (start 197.104 50.292) (end 194.962 48.15) (width 0.25) (layer "B.Cu") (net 5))
 (segment (start 159.004 43.18) (end 165.354 43.18) (width 0.25) (layer "B.Cu") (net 5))
 (segment (start 194.9481 83.0515) (end 195.0466 83.0515) (width 0.25) (layer "B.Cu") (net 5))
 (segment (start 196.85 45.974) (end 199.325 48.449) (width 0.25) (layer "B.Cu") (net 5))
 (segment (start 197.104 53.34) (end 197.104 50.292) (width 0.25) (layer "B.Cu") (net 5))
 (segment (start 136.595201 50.0015) (end 136.885701 50.292) (width 0.25) (layer "B.Cu") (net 5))
 (segment (start 199.325 78.7731) (end 195.0466 83.0515) (width 0.25) (layer "B.Cu") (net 5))
 (segment (start 197.866 48.768) (end 196.596 47.498) (width 0.25) (layer "B.Cu") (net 41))
 (segment (start 159.7152 46.6852) (end 159.7152 44.9072) (width 0.25) (layer "B.Cu") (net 41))
 (segment (start 195.0466 57.6515) (end 197.3485 57.6515) (width 0.25) (layer "B.Cu") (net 41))
 (segment (start 197.866 57.134) (end 197.866 48.768) (width 0.25) (layer "B.Cu") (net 41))
 (segment (start 160.528 47.498) (end 159.7152 46.6852) (width 0.25) (layer "B.Cu") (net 41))
 (segment (start 197.3485 57.6515) (end 197.866 57.134) (width 0.25) (layer "B.Cu") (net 41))
 (segment (start 196.596 47.498) (end 160.528 47.498) (width 0.25) (layer "B.Cu") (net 41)))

